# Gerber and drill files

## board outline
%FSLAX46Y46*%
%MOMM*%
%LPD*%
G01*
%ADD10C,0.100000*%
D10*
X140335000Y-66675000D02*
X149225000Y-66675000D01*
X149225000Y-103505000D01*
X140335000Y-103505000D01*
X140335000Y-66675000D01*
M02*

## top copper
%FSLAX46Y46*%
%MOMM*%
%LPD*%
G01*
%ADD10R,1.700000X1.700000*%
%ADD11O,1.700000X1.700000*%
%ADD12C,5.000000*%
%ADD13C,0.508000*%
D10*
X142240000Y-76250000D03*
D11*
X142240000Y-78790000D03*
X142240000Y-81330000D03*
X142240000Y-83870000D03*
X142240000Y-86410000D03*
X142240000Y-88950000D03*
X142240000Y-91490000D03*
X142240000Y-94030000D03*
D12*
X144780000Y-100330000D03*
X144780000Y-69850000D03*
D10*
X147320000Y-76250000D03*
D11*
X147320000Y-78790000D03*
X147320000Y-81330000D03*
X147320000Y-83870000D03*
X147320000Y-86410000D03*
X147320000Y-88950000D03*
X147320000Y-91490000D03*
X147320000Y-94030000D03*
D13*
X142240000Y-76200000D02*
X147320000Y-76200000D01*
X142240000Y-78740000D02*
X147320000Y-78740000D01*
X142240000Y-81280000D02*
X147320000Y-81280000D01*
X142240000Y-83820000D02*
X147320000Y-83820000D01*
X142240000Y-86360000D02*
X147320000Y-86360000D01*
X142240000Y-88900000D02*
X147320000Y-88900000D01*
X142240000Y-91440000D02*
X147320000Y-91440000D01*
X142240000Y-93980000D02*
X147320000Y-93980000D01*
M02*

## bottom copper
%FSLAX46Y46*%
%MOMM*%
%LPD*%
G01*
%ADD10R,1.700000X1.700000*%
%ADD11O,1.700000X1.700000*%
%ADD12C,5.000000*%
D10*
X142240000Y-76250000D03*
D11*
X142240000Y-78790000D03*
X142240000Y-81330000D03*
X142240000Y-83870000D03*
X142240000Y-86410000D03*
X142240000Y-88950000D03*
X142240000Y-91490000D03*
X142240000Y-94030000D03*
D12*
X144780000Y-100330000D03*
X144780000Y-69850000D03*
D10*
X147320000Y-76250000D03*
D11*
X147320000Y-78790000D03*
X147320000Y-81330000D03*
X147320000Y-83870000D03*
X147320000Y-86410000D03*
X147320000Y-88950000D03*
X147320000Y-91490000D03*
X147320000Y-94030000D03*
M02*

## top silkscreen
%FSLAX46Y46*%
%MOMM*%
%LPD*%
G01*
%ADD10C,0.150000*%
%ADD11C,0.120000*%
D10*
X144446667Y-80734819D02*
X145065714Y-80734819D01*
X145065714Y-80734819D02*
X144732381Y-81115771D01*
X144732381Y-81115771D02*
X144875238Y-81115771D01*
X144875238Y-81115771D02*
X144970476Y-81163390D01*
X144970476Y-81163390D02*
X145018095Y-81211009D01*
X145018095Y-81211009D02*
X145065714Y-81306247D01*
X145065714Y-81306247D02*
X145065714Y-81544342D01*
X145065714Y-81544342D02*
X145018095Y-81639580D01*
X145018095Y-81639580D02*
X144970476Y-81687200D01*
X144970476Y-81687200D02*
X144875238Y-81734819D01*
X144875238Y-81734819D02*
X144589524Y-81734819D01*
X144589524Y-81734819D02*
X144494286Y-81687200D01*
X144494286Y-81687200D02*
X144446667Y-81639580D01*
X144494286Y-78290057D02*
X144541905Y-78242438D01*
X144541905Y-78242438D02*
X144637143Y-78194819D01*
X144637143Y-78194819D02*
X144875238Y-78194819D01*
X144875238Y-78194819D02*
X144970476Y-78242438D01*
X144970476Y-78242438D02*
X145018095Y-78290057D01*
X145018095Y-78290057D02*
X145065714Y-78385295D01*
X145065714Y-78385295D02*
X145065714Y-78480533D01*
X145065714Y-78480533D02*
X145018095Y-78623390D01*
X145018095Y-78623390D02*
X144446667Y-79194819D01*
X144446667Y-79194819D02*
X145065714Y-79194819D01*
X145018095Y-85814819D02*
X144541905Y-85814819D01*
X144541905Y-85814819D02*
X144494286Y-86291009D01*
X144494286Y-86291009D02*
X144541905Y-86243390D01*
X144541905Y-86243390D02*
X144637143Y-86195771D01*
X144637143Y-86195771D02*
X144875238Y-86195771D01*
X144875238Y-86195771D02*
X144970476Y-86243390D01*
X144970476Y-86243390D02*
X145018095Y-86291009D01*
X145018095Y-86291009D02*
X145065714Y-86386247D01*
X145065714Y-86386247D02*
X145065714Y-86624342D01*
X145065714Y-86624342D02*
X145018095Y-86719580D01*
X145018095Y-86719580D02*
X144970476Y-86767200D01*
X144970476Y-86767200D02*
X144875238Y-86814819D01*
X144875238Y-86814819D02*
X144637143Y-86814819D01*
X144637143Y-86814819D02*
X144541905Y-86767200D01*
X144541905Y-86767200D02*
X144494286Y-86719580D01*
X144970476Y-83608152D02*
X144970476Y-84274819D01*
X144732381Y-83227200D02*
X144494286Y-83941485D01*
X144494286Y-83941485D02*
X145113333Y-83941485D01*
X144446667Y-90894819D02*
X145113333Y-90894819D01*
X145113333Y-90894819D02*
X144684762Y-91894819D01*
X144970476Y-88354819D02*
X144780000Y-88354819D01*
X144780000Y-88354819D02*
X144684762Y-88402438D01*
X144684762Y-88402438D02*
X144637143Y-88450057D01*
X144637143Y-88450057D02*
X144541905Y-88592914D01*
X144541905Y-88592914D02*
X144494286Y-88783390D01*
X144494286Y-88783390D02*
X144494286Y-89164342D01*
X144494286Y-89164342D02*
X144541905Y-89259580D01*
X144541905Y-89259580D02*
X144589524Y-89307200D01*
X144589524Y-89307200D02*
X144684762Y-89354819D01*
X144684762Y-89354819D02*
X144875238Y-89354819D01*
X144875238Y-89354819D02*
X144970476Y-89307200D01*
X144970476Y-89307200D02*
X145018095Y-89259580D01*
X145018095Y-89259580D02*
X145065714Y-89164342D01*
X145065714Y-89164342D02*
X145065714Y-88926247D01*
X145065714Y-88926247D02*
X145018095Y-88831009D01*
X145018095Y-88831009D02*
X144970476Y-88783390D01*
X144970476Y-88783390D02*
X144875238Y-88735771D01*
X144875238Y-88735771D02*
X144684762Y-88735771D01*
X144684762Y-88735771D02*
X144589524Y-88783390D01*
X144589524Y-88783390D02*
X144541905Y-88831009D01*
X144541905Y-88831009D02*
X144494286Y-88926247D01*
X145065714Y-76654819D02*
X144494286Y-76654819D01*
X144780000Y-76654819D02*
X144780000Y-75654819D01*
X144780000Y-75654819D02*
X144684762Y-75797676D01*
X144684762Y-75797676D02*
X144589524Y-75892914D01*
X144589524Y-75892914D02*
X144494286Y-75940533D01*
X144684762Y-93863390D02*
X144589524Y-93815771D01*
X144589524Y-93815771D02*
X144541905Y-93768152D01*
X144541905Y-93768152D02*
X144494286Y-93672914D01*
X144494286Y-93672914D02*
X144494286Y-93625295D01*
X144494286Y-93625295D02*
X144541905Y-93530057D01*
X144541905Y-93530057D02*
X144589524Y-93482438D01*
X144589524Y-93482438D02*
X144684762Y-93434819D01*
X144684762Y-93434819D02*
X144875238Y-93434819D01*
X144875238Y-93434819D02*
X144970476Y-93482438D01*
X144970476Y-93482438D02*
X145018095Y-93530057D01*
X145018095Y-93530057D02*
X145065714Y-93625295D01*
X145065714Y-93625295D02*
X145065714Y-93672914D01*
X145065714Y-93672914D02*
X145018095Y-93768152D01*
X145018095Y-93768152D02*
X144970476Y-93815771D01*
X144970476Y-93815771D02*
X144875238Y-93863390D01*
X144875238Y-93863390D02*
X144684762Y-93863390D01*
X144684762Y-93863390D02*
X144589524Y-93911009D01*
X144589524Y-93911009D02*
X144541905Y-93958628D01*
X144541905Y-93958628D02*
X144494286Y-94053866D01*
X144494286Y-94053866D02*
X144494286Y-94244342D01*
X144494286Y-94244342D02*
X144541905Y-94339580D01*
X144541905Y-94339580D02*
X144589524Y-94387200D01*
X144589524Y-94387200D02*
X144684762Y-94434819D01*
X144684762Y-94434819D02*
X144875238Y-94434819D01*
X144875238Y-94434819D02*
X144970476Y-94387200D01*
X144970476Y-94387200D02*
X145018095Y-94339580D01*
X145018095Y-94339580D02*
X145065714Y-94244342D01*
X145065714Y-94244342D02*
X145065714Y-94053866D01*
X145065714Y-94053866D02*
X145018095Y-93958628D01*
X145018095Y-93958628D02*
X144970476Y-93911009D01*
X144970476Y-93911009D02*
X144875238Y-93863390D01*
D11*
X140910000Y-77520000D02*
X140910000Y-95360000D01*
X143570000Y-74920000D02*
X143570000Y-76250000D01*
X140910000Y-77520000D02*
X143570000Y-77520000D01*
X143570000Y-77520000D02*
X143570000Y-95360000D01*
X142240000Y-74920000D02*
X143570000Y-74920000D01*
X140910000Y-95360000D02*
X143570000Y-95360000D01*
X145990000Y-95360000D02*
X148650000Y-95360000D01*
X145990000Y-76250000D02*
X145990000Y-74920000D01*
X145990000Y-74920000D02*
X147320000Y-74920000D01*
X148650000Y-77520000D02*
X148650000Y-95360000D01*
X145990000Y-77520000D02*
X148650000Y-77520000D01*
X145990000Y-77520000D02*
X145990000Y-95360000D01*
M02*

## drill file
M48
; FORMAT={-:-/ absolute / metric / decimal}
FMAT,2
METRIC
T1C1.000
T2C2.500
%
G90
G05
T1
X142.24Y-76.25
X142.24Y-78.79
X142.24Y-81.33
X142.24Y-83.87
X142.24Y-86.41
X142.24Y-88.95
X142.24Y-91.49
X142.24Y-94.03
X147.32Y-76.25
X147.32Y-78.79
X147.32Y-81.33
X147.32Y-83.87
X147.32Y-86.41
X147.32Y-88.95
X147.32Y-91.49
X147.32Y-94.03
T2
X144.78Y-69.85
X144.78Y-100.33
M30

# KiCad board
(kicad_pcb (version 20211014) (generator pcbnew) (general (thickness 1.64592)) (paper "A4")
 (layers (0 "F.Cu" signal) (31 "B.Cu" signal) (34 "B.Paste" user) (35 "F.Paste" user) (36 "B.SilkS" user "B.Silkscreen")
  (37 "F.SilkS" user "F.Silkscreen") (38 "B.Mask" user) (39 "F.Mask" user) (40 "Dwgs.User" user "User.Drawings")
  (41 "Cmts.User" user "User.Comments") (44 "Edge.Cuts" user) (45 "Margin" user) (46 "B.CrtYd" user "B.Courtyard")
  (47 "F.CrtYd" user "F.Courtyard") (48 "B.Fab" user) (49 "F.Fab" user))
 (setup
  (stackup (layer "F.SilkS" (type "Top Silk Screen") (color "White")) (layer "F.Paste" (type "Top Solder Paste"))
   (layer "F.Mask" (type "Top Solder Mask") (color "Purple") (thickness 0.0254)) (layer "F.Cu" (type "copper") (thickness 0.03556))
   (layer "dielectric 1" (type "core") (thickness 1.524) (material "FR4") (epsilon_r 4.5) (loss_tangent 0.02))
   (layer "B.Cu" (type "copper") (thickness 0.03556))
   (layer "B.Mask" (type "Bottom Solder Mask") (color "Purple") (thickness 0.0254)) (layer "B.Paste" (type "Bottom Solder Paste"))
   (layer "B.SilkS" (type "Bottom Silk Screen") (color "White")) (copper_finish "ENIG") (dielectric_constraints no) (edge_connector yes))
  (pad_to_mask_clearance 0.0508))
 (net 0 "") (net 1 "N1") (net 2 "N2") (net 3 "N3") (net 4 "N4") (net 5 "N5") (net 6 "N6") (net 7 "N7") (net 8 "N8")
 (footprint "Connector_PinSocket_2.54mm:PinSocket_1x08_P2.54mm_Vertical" (layer "F.Cu") (at 142.24 76.25)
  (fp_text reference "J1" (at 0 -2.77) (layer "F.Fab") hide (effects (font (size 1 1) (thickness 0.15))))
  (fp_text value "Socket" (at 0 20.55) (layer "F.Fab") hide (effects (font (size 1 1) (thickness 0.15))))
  (fp_line (start -1.33 1.27) (end -1.33 19.11) (layer "F.SilkS") (width 0.12))
  (fp_line (start 1.33 -1.33) (end 1.33 0) (layer "F.SilkS") (width 0.12))
  (fp_line (start -1.33 1.27) (end 1.33 1.27) (layer "F.SilkS") (width 0.12))
  (fp_line (start 1.33 1.27) (end 1.33 19.11) (layer "F.SilkS") (width 0.12))
  (fp_line (start 0 -1.33) (end 1.33 -1.33) (layer "F.SilkS") (width 0.12))
  (fp_line (start -1.33 19.11) (end 1.33 19.11) (layer "F.SilkS") (width 0.12))
  (pad "1" thru_hole rect (at 0 0) (size 1.7 1.7) (drill 1) (layers *.Cu *.Mask) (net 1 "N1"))
  (pad "2" thru_hole oval (at 0 2.54) (size 1.7 1.7) (drill 1) (layers *.Cu *.Mask) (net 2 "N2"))
  (pad "3" thru_hole oval (at 0 5.08) (size 1.7 1.7) (drill 1) (layers *.Cu *.Mask) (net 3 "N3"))
  (pad "4" thru_hole oval (at 0 7.62) (size 1.7 1.7) (drill 1) (layers *.Cu *.Mask) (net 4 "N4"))
  (pad "5" thru_hole oval (at 0 10.16) (size 1.7 1.7) (drill 1) (layers *.Cu *.Mask) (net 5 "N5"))
  (pad "6" thru_hole oval (at 0 12.7) (size 1.7 1.7) (drill 1) (layers *.Cu *.Mask) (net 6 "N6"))
  (pad "7" thru_hole oval (at 0 15.24) (size 1.7 1.7) (drill 1) (layers *.Cu *.Mask) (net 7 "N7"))
  (pad "8" thru_hole oval (at 0 17.78) (size 1.7 1.7) (drill 1) (layers *.Cu *.Mask) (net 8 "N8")))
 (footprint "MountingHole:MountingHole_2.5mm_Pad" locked (layer "F.Cu") (at 144.78 100.33)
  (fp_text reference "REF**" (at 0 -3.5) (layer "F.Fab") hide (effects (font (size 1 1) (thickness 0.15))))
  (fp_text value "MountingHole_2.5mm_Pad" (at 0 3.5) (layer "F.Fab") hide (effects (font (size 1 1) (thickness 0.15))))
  (pad "1" thru_hole circle locked (at 0 0) (size 5 5) (drill 2.5) (layers *.Cu *.Mask)))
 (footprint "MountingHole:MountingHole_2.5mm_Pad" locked (layer "F.Cu") (at 144.78 69.85)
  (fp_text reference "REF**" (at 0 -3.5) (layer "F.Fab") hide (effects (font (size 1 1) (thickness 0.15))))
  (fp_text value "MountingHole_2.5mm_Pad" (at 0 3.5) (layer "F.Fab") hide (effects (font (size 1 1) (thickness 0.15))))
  (pad "1" thru_hole circle locked (at 0 0) (size 5 5) (drill 2.5) (layers *.Cu *.Mask)))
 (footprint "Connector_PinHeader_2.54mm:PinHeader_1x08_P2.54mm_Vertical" (layer "F.Cu") (at 147.32 76.25)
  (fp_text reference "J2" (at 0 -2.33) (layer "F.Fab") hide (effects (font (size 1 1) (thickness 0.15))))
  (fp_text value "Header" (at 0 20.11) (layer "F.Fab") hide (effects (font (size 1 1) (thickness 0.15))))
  (fp_line (start -1.33 19.11) (end 1.33 19.11) (layer "F.SilkS") (width 0.12))
  (fp_line (start -1.33 0) (end -1.33 -1.33) (layer "F.SilkS") (width 0.12))
  (fp_line (start -1.33 -1.33) (end 0 -1.33) (layer "F.SilkS") (width 0.12))
  (fp_line (start 1.33 1.27) (end 1.33 19.11) (layer "F.SilkS") (width 0.12))
  (fp_line (start -1.33 1.27) (end 1.33 1.27) (layer "F.SilkS") (width 0.12))
  (fp_line (start -1.33 1.27) (end -1.33 19.11) (layer "F.SilkS") (width 0.12))
  (pad "1" thru_hole rect (at 0 0) (size 1.7 1.7) (drill 1) (layers *.Cu *.Mask) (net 1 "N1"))
  (pad "2" thru_hole oval (at 0 2.54) (size 1.7 1.7) (drill 1) (layers *.Cu *.Mask) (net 2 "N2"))
  (pad "3" thru_hole oval (at 0 5.08) (size 1.7 1.7) (drill 1) (layers *.Cu *.Mask) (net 3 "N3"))
  (pad "4" thru_hole oval (at 0 7.62) (size 1.7 1.7) (drill 1) (layers *.Cu *.Mask) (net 4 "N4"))
  (pad "5" thru_hole oval (at 0 10.16) (size 1.7 1.7) (drill 1) (layers *.Cu *.Mask) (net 5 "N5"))
  (pad "6" thru_hole oval (at 0 12.7) (size 1.7 1.7) (drill 1) (layers *.Cu *.Mask) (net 6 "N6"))
  (pad "7" thru_hole oval (at 0 15.24) (size 1.7 1.7) (drill 1) (layers *.Cu *.Mask) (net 7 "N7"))
  (pad "8" thru_hole oval (at 0 17.78) (size 1.7 1.7) (drill 1) (layers *.Cu *.Mask) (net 8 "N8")))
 (gr_rect (start 140.335 66.675) (end 149.225 103.505) (layer "Edge.Cuts") (width 0.1) (fill none))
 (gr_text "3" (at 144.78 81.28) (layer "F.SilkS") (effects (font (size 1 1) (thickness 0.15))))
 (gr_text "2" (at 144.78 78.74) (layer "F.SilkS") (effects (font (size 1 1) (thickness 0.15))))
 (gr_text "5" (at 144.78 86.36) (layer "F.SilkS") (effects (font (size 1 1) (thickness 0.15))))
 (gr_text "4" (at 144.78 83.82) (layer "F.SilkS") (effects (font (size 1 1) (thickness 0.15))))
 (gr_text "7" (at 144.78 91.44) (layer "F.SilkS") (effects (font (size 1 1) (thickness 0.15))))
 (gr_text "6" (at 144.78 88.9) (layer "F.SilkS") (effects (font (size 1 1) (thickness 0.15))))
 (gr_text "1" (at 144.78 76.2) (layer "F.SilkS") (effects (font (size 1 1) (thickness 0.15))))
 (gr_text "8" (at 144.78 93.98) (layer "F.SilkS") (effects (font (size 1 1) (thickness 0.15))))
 (segment (start 142.24 76.2) (end 147.32 76.2) (width 0.508) (layer "F.Cu") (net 1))
 (segment (start 142.24 78.74) (end 147.32 78.74) (width 0.508) (layer "F.Cu") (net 2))
 (segment (start 142.24 81.28) (end 147.32 81.28) (width 0.508) (layer "F.Cu") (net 3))
 (segment (start 142.24 83.82) (end 147.32 83.82) (width 0.508) (layer "F.Cu") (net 4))
 (segment (start 142.24 86.36) (end 147.32 86.36) (width 0.508) (layer "F.Cu") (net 5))
 (segment (start 142.24 88.9) (end 147.32 88.9) (width 0.508) (layer "F.Cu") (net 6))
 (segment (start 142.24 91.44) (end 147.32 91.44) (width 0.508) (layer "F.Cu") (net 7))
 (segment (start 142.24 93.98) (end 147.32 93.98) (width 0.508) (layer "F.Cu") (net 8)))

